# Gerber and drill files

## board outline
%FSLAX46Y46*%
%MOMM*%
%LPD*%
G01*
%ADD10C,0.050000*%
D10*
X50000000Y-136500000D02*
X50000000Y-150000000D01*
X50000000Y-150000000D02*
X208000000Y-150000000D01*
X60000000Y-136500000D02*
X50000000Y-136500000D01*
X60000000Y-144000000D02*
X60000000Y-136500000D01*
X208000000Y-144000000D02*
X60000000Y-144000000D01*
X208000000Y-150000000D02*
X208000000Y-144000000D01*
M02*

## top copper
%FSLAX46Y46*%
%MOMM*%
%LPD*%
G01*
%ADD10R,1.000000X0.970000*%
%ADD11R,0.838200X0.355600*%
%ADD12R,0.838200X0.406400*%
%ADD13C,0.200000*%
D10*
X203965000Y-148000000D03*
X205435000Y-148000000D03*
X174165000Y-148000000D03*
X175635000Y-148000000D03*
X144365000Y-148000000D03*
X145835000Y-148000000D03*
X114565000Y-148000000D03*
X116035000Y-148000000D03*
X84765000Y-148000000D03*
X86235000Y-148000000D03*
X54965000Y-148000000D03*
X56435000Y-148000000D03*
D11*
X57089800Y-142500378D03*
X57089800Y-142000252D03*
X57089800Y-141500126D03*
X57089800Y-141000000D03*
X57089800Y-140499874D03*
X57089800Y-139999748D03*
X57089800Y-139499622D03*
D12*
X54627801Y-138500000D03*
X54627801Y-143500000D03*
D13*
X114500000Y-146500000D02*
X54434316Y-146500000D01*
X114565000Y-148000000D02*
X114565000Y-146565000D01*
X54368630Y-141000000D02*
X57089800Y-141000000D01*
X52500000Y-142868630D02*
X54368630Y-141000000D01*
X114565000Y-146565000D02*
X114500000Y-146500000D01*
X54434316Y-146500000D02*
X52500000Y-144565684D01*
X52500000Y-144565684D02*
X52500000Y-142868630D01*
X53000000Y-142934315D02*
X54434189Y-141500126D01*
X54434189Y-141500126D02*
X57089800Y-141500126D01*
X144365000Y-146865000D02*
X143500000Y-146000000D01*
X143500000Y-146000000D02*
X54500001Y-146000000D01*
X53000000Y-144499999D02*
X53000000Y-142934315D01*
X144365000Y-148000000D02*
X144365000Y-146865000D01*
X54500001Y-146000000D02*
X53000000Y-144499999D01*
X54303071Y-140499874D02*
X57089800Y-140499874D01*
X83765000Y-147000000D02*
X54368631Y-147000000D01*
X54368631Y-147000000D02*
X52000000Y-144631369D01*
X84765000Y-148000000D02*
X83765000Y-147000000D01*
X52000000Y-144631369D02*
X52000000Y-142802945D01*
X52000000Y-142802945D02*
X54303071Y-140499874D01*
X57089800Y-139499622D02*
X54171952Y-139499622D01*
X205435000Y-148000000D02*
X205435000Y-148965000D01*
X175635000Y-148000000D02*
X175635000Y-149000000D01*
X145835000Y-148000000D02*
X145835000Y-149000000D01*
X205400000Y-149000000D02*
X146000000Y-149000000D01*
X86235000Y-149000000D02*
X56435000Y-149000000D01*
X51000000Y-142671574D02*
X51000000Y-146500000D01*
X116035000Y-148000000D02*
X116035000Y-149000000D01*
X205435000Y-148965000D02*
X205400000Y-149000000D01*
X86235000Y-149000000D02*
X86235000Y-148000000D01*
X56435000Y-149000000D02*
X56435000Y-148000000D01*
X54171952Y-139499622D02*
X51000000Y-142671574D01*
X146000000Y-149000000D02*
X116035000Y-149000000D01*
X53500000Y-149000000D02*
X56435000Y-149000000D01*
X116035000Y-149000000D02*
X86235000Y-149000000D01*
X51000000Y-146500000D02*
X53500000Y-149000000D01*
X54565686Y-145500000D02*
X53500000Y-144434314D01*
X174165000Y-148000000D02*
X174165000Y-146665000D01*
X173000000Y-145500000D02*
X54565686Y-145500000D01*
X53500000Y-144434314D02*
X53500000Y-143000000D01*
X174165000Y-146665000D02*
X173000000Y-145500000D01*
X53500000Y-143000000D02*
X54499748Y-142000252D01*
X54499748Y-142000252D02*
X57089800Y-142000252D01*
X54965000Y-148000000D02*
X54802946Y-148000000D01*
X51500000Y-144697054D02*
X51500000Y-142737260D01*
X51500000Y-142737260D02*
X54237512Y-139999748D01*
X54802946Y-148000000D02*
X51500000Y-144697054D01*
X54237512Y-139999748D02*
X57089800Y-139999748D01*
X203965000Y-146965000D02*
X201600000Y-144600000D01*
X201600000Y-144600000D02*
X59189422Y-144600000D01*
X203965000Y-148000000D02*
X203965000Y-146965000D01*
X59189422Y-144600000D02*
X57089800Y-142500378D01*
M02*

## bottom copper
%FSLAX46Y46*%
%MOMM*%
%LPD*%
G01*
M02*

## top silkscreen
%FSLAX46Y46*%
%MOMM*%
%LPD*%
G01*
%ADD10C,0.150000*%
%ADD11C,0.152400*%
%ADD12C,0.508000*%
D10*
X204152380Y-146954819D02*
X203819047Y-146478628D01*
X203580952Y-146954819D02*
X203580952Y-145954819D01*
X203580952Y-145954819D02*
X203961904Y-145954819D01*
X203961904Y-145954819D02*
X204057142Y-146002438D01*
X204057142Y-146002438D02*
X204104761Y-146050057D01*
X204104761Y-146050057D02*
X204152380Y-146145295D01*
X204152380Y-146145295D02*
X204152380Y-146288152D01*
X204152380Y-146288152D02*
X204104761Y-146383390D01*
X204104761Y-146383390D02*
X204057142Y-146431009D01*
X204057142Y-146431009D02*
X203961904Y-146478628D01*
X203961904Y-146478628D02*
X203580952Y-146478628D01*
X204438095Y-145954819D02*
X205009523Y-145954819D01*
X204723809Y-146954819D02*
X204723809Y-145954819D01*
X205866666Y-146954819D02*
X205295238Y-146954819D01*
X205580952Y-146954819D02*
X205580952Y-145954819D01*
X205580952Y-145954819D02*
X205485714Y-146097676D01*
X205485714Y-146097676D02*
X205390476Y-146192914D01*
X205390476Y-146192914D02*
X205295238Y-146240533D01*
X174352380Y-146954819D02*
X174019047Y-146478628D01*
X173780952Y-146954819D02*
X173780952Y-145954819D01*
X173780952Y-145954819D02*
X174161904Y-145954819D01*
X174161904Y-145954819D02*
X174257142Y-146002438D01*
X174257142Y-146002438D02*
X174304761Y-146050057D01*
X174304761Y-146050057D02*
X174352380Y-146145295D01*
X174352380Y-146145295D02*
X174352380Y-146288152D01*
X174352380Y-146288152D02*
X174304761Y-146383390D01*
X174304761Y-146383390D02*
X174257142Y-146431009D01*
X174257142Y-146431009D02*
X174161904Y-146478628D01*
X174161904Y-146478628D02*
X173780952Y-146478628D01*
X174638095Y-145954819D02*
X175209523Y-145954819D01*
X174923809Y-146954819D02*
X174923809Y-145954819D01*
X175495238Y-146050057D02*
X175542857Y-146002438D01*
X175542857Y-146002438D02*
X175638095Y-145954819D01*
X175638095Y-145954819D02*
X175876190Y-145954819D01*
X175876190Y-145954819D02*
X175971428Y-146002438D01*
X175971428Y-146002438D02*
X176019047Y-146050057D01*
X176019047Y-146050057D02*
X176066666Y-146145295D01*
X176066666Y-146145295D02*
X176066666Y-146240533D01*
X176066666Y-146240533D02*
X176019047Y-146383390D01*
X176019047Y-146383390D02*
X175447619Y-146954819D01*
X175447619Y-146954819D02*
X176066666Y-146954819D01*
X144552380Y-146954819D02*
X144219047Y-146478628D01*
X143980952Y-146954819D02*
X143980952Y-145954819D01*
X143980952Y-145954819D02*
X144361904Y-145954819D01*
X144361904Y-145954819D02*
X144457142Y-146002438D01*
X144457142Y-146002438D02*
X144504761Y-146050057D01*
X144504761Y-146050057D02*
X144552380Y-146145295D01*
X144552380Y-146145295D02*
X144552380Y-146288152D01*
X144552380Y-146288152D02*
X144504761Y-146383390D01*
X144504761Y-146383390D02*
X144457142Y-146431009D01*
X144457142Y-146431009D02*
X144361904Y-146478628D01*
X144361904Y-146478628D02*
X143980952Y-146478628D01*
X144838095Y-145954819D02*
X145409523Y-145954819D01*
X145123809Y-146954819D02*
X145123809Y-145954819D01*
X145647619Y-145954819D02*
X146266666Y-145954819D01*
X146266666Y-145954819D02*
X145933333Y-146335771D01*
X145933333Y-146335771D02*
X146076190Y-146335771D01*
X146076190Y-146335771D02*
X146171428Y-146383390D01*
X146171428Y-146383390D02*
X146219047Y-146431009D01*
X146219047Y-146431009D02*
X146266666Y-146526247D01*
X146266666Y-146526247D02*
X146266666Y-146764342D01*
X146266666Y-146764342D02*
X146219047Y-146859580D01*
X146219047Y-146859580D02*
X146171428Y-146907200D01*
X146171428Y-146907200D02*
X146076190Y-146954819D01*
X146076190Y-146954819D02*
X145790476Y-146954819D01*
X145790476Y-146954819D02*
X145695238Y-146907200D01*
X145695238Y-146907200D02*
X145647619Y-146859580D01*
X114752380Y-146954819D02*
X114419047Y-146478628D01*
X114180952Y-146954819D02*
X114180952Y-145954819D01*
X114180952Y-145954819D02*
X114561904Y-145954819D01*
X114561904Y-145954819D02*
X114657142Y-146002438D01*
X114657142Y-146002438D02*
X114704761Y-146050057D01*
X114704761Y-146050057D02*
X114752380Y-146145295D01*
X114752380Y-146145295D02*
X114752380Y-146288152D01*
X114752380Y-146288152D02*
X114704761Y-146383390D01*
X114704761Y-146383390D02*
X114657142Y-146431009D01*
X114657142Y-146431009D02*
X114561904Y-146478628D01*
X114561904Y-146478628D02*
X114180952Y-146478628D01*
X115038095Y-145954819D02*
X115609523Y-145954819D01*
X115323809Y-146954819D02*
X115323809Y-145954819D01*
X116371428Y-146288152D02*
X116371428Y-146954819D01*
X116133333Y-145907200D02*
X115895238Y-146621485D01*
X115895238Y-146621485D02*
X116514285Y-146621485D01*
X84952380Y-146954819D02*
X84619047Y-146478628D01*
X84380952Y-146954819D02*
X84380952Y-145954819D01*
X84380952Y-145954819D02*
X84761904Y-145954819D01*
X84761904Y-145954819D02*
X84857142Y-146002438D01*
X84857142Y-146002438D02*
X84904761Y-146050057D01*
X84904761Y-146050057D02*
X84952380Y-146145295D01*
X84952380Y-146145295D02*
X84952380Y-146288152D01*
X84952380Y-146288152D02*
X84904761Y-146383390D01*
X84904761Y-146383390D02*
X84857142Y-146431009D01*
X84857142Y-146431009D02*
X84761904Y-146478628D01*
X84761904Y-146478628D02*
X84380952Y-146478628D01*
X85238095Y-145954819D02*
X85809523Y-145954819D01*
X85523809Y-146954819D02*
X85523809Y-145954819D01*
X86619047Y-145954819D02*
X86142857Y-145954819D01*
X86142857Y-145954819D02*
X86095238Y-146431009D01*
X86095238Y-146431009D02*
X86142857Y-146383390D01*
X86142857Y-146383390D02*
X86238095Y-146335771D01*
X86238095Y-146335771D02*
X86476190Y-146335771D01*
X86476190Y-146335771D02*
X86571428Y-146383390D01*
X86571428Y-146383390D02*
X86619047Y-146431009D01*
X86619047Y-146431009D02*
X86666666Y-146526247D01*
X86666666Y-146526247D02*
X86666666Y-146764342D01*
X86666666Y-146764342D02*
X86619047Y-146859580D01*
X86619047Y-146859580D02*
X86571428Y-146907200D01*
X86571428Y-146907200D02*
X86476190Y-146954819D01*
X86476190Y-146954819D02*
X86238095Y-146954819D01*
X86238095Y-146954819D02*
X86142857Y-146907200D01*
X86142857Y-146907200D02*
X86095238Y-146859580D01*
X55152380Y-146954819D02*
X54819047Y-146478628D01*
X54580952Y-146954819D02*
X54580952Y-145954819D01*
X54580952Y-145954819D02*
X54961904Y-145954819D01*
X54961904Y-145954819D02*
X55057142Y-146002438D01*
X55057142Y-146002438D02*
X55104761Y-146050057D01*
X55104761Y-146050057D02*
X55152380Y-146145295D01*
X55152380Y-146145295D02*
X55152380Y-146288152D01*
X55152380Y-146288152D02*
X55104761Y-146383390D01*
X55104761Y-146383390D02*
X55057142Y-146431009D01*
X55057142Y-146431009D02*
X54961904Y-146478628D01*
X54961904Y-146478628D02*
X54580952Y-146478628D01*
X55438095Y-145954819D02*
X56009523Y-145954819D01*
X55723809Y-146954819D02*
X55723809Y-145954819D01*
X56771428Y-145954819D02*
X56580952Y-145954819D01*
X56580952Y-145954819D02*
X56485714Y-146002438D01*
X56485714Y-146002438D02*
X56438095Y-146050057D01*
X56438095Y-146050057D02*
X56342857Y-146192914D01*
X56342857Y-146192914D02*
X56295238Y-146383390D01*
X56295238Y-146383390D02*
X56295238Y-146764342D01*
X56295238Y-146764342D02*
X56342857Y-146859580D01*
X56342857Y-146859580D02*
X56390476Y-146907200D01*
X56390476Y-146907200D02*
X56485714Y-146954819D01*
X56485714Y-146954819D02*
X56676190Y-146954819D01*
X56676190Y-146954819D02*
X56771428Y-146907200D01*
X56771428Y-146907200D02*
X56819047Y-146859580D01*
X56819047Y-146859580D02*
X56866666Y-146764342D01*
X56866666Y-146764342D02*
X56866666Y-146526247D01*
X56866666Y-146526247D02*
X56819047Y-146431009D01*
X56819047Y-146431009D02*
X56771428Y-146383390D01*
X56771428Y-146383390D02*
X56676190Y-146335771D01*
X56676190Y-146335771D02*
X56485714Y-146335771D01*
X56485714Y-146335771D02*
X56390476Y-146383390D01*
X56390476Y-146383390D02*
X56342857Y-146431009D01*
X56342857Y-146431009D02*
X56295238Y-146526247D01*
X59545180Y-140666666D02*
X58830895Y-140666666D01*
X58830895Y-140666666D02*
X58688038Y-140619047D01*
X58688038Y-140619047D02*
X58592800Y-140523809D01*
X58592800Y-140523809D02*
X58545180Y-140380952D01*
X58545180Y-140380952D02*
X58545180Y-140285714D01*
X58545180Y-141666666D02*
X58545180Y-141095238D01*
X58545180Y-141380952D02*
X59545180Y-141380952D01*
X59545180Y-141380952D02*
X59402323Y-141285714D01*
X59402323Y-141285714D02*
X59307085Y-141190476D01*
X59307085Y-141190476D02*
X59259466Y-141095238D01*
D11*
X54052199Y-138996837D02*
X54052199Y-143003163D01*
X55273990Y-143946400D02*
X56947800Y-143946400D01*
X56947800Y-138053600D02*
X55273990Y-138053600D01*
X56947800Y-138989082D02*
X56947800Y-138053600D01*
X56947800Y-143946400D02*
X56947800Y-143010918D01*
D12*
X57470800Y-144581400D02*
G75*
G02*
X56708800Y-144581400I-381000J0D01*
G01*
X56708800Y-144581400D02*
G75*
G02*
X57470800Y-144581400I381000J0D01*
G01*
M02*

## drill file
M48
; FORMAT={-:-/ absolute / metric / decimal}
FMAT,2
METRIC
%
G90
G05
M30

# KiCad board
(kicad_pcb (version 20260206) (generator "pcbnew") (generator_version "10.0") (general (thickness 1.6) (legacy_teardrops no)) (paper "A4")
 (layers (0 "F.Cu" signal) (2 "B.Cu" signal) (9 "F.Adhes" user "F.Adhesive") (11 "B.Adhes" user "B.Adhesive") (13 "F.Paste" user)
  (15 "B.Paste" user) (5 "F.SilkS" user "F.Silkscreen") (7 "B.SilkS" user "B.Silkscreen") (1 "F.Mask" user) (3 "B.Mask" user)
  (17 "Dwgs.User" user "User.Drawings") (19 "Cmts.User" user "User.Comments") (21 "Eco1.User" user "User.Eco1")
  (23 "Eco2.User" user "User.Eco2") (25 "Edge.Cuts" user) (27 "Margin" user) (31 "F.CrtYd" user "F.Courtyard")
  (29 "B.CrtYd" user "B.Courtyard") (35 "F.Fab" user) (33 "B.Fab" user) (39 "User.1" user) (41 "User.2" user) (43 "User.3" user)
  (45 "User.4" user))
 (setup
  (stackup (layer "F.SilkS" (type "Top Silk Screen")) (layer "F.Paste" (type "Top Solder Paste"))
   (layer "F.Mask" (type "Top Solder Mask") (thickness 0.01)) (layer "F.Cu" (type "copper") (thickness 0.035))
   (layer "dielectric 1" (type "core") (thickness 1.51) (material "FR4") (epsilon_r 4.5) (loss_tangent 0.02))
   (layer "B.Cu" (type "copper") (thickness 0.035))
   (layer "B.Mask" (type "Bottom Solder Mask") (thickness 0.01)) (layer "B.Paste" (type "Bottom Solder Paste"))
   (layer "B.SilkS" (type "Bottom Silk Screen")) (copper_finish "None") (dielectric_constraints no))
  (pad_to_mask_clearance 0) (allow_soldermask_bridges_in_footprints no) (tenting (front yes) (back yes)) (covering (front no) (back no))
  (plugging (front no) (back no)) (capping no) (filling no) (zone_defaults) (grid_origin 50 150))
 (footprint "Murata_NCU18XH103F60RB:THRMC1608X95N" (layer "F.Cu") (at 204.7 148)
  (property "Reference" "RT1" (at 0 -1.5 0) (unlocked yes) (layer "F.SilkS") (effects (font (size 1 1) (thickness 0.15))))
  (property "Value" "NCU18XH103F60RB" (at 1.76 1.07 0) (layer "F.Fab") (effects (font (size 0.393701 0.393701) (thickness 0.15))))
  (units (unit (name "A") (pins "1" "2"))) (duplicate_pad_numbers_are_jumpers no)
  (pad "1" smd rect (at -0.735 0) (size 1 0.97) (layers "F.Cu" "F.Mask" "F.Paste") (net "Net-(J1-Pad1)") (solder_mask_margin 0.102))
  (pad "2" smd rect (at 0.735 0) (size 1 0.97) (layers "F.Cu" "F.Mask" "F.Paste") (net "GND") (solder_mask_margin 0.102)))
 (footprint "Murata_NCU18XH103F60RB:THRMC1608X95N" (layer "F.Cu") (at 174.9 148)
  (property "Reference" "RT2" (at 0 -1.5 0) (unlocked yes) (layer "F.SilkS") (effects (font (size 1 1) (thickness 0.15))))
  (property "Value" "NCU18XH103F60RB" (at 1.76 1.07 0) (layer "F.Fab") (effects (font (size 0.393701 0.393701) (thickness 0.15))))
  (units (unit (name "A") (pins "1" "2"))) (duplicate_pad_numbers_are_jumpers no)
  (pad "1" smd rect (at -0.735 0) (size 1 0.97) (layers "F.Cu" "F.Mask" "F.Paste") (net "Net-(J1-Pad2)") (solder_mask_margin 0.102))
  (pad "2" smd rect (at 0.735 0) (size 1 0.97) (layers "F.Cu" "F.Mask" "F.Paste") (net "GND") (solder_mask_margin 0.102)))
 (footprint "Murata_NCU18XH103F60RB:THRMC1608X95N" (layer "F.Cu") (at 145.1 148)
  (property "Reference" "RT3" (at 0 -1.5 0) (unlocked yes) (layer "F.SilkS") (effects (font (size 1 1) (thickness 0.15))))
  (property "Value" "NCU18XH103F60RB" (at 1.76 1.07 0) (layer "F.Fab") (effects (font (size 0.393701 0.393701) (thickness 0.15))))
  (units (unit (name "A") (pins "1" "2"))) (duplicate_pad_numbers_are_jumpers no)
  (pad "1" smd rect (at -0.735 0) (size 1 0.97) (layers "F.Cu" "F.Mask" "F.Paste") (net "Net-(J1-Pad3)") (solder_mask_margin 0.102))
  (pad "2" smd rect (at 0.735 0) (size 1 0.97) (layers "F.Cu" "F.Mask" "F.Paste") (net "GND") (solder_mask_margin 0.102)))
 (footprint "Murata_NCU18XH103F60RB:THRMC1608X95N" (layer "F.Cu") (at 115.3 148)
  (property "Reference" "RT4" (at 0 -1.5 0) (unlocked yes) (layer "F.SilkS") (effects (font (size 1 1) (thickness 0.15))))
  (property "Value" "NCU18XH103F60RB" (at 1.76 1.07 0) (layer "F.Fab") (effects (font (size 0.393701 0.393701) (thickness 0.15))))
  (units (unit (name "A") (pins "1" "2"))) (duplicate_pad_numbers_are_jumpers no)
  (pad "1" smd rect (at -0.735 0) (size 1 0.97) (layers "F.Cu" "F.Mask" "F.Paste") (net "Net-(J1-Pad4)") (solder_mask_margin 0.102))
  (pad "2" smd rect (at 0.735 0) (size 1 0.97) (layers "F.Cu" "F.Mask" "F.Paste") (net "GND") (solder_mask_margin 0.102)))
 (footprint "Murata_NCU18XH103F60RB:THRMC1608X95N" (layer "F.Cu") (at 85.5 148)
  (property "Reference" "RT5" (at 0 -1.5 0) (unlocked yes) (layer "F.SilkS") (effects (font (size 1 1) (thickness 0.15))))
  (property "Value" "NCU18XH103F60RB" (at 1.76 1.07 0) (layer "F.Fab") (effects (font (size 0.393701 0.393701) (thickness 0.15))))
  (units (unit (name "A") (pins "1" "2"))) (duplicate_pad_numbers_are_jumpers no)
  (pad "1" smd rect (at -0.735 0) (size 1 0.97) (layers "F.Cu" "F.Mask" "F.Paste") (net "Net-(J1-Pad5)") (solder_mask_margin 0.102))
  (pad "2" smd rect (at 0.735 0) (size 1 0.97) (layers "F.Cu" "F.Mask" "F.Paste") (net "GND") (solder_mask_margin 0.102)))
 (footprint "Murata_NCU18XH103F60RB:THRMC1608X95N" (layer "F.Cu") (at 55.7 148)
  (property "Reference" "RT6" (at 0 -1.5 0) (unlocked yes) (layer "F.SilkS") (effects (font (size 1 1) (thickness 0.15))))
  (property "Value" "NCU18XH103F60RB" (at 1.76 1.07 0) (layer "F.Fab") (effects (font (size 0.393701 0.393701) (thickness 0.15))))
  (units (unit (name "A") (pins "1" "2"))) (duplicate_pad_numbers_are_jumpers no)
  (pad "1" smd rect (at -0.735 0) (size 1 0.97) (layers "F.Cu" "F.Mask" "F.Paste") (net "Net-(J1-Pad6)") (solder_mask_margin 0.102))
  (pad "2" smd rect (at 0.735 0) (size 1 0.97) (layers "F.Cu" "F.Mask" "F.Paste") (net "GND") (solder_mask_margin 0.102)))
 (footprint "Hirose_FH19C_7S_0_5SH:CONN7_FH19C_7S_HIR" (layer "F.Cu") (at 55.5 141 -90)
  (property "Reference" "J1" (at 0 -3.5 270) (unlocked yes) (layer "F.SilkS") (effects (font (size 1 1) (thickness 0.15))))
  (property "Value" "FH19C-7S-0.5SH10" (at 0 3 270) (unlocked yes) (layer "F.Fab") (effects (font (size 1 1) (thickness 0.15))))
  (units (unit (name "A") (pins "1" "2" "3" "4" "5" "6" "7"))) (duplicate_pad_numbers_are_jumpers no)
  (fp_line (start -2.003163 1.447801) (end 2.003163 1.447801) (stroke (width 0.1524) (type solid)) (layer "F.SilkS"))
  (fp_line (start 2.9464 0.22601) (end 2.9464 -1.4478) (stroke (width 0.1524) (type solid)) (layer "F.SilkS"))
  (fp_line (start -2.9464 -1.4478) (end -2.9464 0.22601) (stroke (width 0.1524) (type solid)) (layer "F.SilkS"))
  (fp_line (start -2.010918 -1.4478) (end -2.9464 -1.4478) (stroke (width 0.1524) (type solid)) (layer "F.SilkS"))
  (fp_line (start 2.9464 -1.4478) (end 2.010918 -1.4478) (stroke (width 0.1524) (type solid)) (layer "F.SilkS"))
  (fp_circle (center 3.5814 -1.5898) (end 3.9624 -1.5898) (stroke (width 0.508) (type solid)) (fill no) (layer "F.SilkS"))
  (pad "1" smd rect (at 1.500378 -1.5898 270) (size 0.3556 0.8382) (layers "F.Cu" "F.Mask" "F.Paste") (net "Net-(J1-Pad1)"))
  (pad "2" smd rect (at 1.000252 -1.5898 270) (size 0.3556 0.8382) (layers "F.Cu" "F.Mask" "F.Paste") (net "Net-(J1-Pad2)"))
  (pad "3" smd rect (at 0.500126 -1.5898 270) (size 0.3556 0.8382) (layers "F.Cu" "F.Mask" "F.Paste") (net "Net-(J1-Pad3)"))
  (pad "4" smd rect (at 0 -1.5898 270) (size 0.3556 0.8382) (layers "F.Cu" "F.Mask" "F.Paste") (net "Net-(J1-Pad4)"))
  (pad "5" smd rect (at -0.500126 -1.5898 270) (size 0.3556 0.8382) (layers "F.Cu" "F.Mask" "F.Paste") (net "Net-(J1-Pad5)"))
  (pad "6" smd rect (at -1.000252 -1.5898 270) (size 0.3556 0.8382) (layers "F.Cu" "F.Mask" "F.Paste") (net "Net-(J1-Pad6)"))
  (pad "7" smd rect (at -1.500378 -1.5898 270) (size 0.3556 0.8382) (layers "F.Cu" "F.Mask" "F.Paste") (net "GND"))
  (pad "8" smd rect (at -2.5 0.872199 270) (size 0.4064 0.8382) (layers "F.Cu" "F.Mask" "F.Paste"))
  (pad "9" smd rect (at 2.5 0.872199 270) (size 0.4064 0.8382) (layers "F.Cu" "F.Mask" "F.Paste")))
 (gr_line (start 50 136.5) (end 50 150) (stroke (width 0.05) (type solid)) (layer "Edge.Cuts"))
 (gr_line (start 50 150) (end 208 150) (stroke (width 0.05) (type solid)) (locked yes) (layer "Edge.Cuts"))
 (gr_line (start 60 136.5) (end 50 136.5) (stroke (width 0.05) (type default)) (layer "Edge.Cuts"))
 (gr_line (start 60 144) (end 60 136.5) (stroke (width 0.05) (type default)) (layer "Edge.Cuts"))
 (gr_line (start 208 144) (end 60 144) (stroke (width 0.05) (type default)) (layer "Edge.Cuts"))
 (gr_line (start 208 150) (end 208 144) (stroke (width 0.05) (type default)) (layer "Edge.Cuts"))
 (segment (start 114.5 146.5) (end 54.434316 146.5) (width 0.2) (layer "F.Cu") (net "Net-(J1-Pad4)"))
 (segment (start 114.565 148) (end 114.565 146.565) (width 0.2) (layer "F.Cu") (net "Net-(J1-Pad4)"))
 (segment (start 54.36863 141) (end 57.0898 141) (width 0.2) (layer "F.Cu") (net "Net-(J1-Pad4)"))
 (segment (start 52.5 142.86863) (end 54.36863 141) (width 0.2) (layer "F.Cu") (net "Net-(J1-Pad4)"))
 (segment (start 114.565 146.565) (end 114.5 146.5) (width 0.2) (layer "F.Cu") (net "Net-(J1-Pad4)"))
 (segment (start 54.434316 146.5) (end 52.5 144.565684) (width 0.2) (layer "F.Cu") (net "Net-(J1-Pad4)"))
 (segment (start 52.5 144.565684) (end 52.5 142.86863) (width 0.2) (layer "F.Cu") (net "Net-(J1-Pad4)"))
 (segment (start 53 142.934315) (end 54.434189 141.500126) (width 0.2) (layer "F.Cu") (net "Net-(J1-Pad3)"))
 (segment (start 54.434189 141.500126) (end 57.0898 141.500126) (width 0.2) (layer "F.Cu") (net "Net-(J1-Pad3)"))
 (segment (start 144.365 146.865) (end 143.5 146) (width 0.2) (layer "F.Cu") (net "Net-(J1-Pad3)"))
 (segment (start 143.5 146) (end 54.500001 146) (width 0.2) (layer "F.Cu") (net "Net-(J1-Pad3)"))
 (segment (start 53 144.499999) (end 53 142.934315) (width 0.2) (layer "F.Cu") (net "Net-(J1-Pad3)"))
 (segment (start 144.365 148) (end 144.365 146.865) (width 0.2) (layer "F.Cu") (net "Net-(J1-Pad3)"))
 (segment (start 54.500001 146) (end 53 144.499999) (width 0.2) (layer "F.Cu") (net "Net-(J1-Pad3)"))
 (segment (start 54.303071 140.499874) (end 57.0898 140.499874) (width 0.2) (layer "F.Cu") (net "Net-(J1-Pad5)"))
 (segment (start 83.765 147) (end 54.368631 147) (width 0.2) (layer "F.Cu") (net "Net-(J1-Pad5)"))
 (segment (start 54.368631 147) (end 52 144.631369) (width 0.2) (layer "F.Cu") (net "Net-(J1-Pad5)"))
 (segment (start 84.765 148) (end 83.765 147) (width 0.2) (layer "F.Cu") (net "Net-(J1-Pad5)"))
 (segment (start 52 144.631369) (end 52 142.802945) (width 0.2) (layer "F.Cu") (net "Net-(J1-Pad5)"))
 (segment (start 52 142.802945) (end 54.303071 140.499874) (width 0.2) (layer "F.Cu") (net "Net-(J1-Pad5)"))
 (segment (start 57.0898 139.499622) (end 54.171952 139.499622) (width 0.2) (layer "F.Cu") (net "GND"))
 (segment (start 205.435 148) (end 205.435 148.965) (width 0.2) (layer "F.Cu") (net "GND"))
 (segment (start 175.635 148) (end 175.635 149) (width 0.2) (layer "F.Cu") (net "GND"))
 (segment (start 145.835 148) (end 145.835 149) (width 0.2) (layer "F.Cu") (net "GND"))
 (segment (start 205.4 149) (end 146 149) (width 0.2) (layer "F.Cu") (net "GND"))
 (segment (start 86.235 149) (end 56.435 149) (width 0.2) (layer "F.Cu") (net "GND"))
 (segment (start 51 142.671574) (end 51 146.5) (width 0.2) (layer "F.Cu") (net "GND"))
 (segment (start 116.035 148) (end 116.035 149) (width 0.2) (layer "F.Cu") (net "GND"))
 (segment (start 205.435 148.965) (end 205.4 149) (width 0.2) (layer "F.Cu") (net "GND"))
 (segment (start 86.235 149) (end 86.235 148) (width 0.2) (layer "F.Cu") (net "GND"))
 (segment (start 56.435 149) (end 56.435 148) (width 0.2) (layer "F.Cu") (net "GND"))
 (segment (start 54.171952 139.499622) (end 51 142.671574) (width 0.2) (layer "F.Cu") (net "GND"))
 (segment (start 146 149) (end 116.035 149) (width 0.2) (layer "F.Cu") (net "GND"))
 (segment (start 53.5 149) (end 56.435 149) (width 0.2) (layer "F.Cu") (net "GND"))
 (segment (start 116.035 149) (end 86.235 149) (width 0.2) (layer "F.Cu") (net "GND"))
 (segment (start 51 146.5) (end 53.5 149) (width 0.2) (layer "F.Cu") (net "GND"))
 (segment (start 54.565686 145.5) (end 53.5 144.434314) (width 0.2) (layer "F.Cu") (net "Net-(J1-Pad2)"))
 (segment (start 174.165 148) (end 174.165 146.665) (width 0.2) (layer "F.Cu") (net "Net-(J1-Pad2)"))
 (segment (start 173 145.5) (end 54.565686 145.5) (width 0.2) (layer "F.Cu") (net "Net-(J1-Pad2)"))
 (segment (start 53.5 144.434314) (end 53.5 143) (width 0.2) (layer "F.Cu") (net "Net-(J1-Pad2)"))
 (segment (start 174.165 146.665) (end 173 145.5) (width 0.2) (layer "F.Cu") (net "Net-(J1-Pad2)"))
 (segment (start 53.5 143) (end 54.499748 142.000252) (width 0.2) (layer "F.Cu") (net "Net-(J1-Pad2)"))
 (segment (start 54.499748 142.000252) (end 57.0898 142.000252) (width 0.2) (layer "F.Cu") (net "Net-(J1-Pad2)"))
 (segment (start 54.965 148) (end 54.802946 148) (width 0.2) (layer "F.Cu") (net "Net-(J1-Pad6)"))
 (segment (start 51.5 144.697054) (end 51.5 142.73726) (width 0.2) (layer "F.Cu") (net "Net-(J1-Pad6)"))
 (segment (start 51.5 142.73726) (end 54.237512 139.999748) (width 0.2) (layer "F.Cu") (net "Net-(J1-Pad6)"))
 (segment (start 54.802946 148) (end 51.5 144.697054) (width 0.2) (layer "F.Cu") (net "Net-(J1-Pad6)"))
 (segment (start 54.237512 139.999748) (end 57.0898 139.999748) (width 0.2) (layer "F.Cu") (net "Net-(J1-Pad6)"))
 (segment (start 203.965 146.965) (end 201.6 144.6) (width 0.2) (layer "F.Cu") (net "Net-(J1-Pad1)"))
 (segment (start 201.6 144.6) (end 59.189422 144.6) (width 0.2) (layer "F.Cu") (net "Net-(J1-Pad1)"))
 (segment (start 203.965 148) (end 203.965 146.965) (width 0.2) (layer "F.Cu") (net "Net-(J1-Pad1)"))
 (segment (start 59.189422 144.6) (end 57.0898 142.500378) (width 0.2) (layer "F.Cu") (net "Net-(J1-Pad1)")))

